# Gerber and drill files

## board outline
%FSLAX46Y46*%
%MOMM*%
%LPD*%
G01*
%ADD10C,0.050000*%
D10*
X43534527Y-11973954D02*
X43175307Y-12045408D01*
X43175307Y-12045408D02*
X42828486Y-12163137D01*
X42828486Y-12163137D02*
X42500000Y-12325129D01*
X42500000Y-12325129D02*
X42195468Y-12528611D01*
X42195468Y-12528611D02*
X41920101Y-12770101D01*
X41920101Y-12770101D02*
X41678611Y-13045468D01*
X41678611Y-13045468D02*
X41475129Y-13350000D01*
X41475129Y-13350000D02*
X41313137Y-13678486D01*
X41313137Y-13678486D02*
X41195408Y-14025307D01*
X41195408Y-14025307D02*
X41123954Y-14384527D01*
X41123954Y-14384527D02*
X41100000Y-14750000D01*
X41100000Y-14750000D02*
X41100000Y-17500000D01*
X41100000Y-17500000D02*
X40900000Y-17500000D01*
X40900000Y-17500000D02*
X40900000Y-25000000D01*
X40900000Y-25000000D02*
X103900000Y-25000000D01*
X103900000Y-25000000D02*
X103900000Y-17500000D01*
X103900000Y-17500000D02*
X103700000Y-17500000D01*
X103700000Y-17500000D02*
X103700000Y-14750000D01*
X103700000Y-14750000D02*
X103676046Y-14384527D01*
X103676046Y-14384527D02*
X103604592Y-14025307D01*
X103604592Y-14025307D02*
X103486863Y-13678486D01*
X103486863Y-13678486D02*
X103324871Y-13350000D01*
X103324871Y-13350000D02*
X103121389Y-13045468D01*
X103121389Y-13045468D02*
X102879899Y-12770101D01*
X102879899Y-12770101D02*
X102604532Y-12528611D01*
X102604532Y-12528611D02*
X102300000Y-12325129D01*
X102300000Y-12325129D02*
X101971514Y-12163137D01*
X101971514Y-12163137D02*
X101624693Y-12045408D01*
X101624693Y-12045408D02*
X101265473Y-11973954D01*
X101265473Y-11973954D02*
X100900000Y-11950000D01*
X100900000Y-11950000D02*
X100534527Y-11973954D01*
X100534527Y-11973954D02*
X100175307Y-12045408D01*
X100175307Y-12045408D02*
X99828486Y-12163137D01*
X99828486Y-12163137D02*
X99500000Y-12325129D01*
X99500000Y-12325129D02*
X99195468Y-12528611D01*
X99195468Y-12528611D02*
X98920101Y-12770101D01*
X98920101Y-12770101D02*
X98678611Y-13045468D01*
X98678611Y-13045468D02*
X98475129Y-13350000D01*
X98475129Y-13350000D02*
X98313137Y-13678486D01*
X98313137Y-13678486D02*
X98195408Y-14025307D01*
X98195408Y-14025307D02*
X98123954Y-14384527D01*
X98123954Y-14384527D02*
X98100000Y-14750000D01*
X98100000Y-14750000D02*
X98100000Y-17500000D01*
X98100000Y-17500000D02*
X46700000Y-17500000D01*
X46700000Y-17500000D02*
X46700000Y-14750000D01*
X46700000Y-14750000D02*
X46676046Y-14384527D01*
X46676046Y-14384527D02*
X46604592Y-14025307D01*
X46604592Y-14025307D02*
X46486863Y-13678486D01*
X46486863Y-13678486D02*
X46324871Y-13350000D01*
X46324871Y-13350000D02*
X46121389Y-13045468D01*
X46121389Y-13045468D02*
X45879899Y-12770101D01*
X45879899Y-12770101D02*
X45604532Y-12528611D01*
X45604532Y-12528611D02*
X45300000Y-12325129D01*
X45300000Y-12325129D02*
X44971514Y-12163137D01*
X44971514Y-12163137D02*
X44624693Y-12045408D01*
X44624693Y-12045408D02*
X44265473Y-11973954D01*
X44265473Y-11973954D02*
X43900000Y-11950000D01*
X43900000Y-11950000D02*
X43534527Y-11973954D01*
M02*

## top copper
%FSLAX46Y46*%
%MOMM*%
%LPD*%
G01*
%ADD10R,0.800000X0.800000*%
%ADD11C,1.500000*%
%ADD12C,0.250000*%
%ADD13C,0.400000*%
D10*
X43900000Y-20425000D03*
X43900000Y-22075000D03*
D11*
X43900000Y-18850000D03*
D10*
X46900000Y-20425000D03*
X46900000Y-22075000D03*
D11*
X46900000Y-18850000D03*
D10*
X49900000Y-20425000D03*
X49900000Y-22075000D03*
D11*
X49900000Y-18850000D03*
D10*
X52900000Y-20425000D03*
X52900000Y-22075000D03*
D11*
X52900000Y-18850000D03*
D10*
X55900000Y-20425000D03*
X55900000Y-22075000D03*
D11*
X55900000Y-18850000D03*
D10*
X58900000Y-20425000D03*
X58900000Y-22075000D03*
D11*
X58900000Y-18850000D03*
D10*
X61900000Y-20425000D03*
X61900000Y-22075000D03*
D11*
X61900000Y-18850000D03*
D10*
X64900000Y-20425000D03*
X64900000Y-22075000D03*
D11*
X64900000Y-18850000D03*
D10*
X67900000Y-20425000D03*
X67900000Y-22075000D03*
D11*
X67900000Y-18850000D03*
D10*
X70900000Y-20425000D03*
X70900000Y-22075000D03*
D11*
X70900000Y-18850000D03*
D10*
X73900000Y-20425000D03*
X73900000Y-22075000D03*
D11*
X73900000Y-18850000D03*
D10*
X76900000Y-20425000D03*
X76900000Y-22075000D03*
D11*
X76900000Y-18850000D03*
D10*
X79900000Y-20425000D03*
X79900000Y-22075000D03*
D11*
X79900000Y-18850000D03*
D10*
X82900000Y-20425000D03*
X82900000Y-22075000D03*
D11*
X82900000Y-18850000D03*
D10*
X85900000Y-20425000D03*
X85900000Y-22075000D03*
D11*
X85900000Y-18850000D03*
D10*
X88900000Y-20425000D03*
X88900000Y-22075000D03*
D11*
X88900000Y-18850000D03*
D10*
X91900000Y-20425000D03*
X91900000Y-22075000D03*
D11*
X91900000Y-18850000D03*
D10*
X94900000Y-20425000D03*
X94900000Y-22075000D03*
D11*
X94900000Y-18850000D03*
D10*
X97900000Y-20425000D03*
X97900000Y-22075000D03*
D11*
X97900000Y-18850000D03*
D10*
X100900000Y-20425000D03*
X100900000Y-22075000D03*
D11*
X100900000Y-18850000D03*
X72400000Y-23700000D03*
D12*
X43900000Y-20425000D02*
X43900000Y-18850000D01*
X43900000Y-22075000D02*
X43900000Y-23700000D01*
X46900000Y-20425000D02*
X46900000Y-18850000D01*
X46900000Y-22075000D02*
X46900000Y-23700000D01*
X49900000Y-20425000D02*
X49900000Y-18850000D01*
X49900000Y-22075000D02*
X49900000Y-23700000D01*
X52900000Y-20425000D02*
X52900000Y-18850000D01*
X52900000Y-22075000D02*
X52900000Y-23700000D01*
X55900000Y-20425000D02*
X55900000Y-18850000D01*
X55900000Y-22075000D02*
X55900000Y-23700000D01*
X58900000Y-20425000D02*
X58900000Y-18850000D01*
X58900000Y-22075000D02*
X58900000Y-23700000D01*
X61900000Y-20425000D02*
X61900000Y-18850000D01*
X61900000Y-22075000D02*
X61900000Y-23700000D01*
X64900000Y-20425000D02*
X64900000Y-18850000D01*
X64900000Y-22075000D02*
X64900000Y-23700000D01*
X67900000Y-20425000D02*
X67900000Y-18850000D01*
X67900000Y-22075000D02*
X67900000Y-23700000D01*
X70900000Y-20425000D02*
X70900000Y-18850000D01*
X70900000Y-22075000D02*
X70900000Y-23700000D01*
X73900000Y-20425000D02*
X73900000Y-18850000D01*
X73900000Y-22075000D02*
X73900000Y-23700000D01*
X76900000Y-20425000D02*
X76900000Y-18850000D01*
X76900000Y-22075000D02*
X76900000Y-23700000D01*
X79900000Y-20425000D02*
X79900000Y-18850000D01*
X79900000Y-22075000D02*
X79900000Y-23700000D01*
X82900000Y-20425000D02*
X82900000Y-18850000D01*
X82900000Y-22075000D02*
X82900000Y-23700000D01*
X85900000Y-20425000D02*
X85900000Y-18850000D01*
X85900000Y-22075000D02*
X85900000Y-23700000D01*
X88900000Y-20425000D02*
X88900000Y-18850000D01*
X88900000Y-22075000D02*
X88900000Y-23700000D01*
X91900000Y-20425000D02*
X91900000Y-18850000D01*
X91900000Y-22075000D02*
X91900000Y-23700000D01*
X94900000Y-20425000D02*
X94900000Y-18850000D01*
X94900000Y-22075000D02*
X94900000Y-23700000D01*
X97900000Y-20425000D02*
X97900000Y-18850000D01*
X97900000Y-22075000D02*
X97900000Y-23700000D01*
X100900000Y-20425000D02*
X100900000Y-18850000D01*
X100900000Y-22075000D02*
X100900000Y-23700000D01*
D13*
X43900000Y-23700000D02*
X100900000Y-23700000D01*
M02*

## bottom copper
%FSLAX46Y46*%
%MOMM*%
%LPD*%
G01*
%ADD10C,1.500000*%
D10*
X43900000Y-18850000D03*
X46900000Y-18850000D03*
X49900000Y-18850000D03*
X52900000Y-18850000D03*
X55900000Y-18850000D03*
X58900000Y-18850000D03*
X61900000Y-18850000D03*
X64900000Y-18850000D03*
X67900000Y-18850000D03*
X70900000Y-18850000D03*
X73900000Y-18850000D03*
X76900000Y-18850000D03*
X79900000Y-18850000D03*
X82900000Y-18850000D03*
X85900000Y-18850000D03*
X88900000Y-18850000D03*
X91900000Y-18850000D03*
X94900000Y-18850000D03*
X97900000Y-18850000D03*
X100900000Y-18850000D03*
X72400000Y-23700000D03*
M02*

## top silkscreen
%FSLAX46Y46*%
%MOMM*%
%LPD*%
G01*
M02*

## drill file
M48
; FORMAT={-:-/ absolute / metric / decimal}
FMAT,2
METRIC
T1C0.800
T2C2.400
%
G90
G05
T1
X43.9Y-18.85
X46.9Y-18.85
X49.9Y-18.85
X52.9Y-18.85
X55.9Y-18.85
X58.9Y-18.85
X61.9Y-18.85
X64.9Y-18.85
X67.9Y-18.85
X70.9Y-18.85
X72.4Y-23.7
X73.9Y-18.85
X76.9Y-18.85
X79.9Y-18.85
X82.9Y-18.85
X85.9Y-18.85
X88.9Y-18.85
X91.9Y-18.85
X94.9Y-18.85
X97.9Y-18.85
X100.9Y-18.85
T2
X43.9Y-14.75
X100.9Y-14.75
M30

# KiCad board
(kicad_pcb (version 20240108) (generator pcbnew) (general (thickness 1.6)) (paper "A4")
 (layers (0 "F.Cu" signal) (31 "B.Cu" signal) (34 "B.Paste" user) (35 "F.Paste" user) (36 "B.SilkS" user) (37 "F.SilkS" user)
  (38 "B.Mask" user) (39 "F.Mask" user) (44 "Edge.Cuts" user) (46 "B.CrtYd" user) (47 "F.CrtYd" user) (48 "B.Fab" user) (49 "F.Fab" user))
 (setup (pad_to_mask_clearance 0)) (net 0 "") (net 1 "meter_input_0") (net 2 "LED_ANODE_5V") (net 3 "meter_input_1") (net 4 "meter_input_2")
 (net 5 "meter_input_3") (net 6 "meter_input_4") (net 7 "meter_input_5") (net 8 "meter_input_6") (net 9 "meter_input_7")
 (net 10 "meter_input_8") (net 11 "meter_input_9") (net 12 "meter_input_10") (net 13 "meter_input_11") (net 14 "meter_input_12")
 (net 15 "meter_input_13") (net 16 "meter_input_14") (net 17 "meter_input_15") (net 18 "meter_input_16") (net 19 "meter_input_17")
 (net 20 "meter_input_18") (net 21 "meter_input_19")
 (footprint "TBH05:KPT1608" (layer "F.Cu") (at 43.9 21.25)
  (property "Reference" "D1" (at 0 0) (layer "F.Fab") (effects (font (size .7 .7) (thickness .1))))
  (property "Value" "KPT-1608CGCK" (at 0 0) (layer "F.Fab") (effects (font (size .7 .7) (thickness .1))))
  (pad "1" smd rect (at 0 -.825) (size .8 .8) (layers "F.Cu" "F.Paste" "F.Mask") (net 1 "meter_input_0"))
  (pad "2" smd rect (at 0 .825) (size .8 .8) (layers "F.Cu" "F.Paste" "F.Mask") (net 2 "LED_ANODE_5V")))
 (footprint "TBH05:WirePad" (layer "F.Cu") (at 43.9 18.85)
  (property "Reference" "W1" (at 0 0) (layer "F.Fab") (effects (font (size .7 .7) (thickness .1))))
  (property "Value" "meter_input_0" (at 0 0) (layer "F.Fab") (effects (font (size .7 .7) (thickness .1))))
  (pad "1" thru_hole circle (at 0 0) (size 1.5 1.5) (drill .8) (layers "*.Cu" "*.Mask") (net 1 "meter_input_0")))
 (segment (start 43.9 20.425) (end 43.9 18.85) (width 0.25) (layer "F.Cu") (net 1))
 (segment (start 43.9 22.075) (end 43.9 23.7) (width 0.25) (layer "F.Cu") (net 2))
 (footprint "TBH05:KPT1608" (layer "F.Cu") (at 46.9 21.25)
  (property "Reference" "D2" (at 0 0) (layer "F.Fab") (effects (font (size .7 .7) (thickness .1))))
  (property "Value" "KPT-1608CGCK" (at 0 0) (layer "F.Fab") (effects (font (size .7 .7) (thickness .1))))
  (pad "1" smd rect (at 0 -.825) (size .8 .8) (layers "F.Cu" "F.Paste" "F.Mask") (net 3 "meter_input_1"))
  (pad "2" smd rect (at 0 .825) (size .8 .8) (layers "F.Cu" "F.Paste" "F.Mask") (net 2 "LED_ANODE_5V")))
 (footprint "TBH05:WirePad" (layer "F.Cu") (at 46.9 18.85)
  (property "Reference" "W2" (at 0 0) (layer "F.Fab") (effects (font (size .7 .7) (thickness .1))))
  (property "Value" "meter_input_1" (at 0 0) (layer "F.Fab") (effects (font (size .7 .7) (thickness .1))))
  (pad "1" thru_hole circle (at 0 0) (size 1.5 1.5) (drill .8) (layers "*.Cu" "*.Mask") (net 3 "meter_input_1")))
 (segment (start 46.9 20.425) (end 46.9 18.85) (width 0.25) (layer "F.Cu") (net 3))
 (segment (start 46.9 22.075) (end 46.9 23.7) (width 0.25) (layer "F.Cu") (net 2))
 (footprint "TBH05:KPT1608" (layer "F.Cu") (at 49.9 21.25)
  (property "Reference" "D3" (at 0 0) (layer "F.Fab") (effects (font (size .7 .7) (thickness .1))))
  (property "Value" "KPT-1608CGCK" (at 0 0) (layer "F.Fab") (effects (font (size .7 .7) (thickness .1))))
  (pad "1" smd rect (at 0 -.825) (size .8 .8) (layers "F.Cu" "F.Paste" "F.Mask") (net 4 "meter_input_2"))
  (pad "2" smd rect (at 0 .825) (size .8 .8) (layers "F.Cu" "F.Paste" "F.Mask") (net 2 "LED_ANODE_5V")))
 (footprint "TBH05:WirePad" (layer "F.Cu") (at 49.9 18.85)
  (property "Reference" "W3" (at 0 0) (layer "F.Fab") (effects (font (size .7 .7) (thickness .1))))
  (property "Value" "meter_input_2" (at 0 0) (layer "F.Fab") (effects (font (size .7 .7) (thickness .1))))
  (pad "1" thru_hole circle (at 0 0) (size 1.5 1.5) (drill .8) (layers "*.Cu" "*.Mask") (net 4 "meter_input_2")))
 (segment (start 49.9 20.425) (end 49.9 18.85) (width 0.25) (layer "F.Cu") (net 4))
 (segment (start 49.9 22.075) (end 49.9 23.7) (width 0.25) (layer "F.Cu") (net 2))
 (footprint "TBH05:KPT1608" (layer "F.Cu") (at 52.9 21.25)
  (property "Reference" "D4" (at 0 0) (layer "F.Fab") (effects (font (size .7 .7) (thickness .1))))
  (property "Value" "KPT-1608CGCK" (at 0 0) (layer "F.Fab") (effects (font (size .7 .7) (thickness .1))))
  (pad "1" smd rect (at 0 -.825) (size .8 .8) (layers "F.Cu" "F.Paste" "F.Mask") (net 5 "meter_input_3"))
  (pad "2" smd rect (at 0 .825) (size .8 .8) (layers "F.Cu" "F.Paste" "F.Mask") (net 2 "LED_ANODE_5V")))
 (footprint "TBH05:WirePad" (layer "F.Cu") (at 52.9 18.85)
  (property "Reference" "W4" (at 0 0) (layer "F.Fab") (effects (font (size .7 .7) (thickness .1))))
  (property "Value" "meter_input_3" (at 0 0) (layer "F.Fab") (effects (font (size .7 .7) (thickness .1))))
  (pad "1" thru_hole circle (at 0 0) (size 1.5 1.5) (drill .8) (layers "*.Cu" "*.Mask") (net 5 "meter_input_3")))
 (segment (start 52.9 20.425) (end 52.9 18.85) (width 0.25) (layer "F.Cu") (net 5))
 (segment (start 52.9 22.075) (end 52.9 23.7) (width 0.25) (layer "F.Cu") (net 2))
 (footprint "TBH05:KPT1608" (layer "F.Cu") (at 55.9 21.25)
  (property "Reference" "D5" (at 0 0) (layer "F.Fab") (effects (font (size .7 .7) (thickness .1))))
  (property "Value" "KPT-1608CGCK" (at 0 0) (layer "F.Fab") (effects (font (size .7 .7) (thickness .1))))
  (pad "1" smd rect (at 0 -.825) (size .8 .8) (layers "F.Cu" "F.Paste" "F.Mask") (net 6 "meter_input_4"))
  (pad "2" smd rect (at 0 .825) (size .8 .8) (layers "F.Cu" "F.Paste" "F.Mask") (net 2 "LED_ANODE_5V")))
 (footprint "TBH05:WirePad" (layer "F.Cu") (at 55.9 18.85)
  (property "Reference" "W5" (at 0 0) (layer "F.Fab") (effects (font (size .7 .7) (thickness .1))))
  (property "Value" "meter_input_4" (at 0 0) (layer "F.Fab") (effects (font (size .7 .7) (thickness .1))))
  (pad "1" thru_hole circle (at 0 0) (size 1.5 1.5) (drill .8) (layers "*.Cu" "*.Mask") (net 6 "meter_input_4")))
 (segment (start 55.9 20.425) (end 55.9 18.85) (width 0.25) (layer "F.Cu") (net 6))
 (segment (start 55.9 22.075) (end 55.9 23.7) (width 0.25) (layer "F.Cu") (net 2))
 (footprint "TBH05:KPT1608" (layer "F.Cu") (at 58.9 21.25)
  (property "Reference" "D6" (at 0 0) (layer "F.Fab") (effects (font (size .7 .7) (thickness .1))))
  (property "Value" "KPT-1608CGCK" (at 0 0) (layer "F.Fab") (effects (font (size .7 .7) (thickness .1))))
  (pad "1" smd rect (at 0 -.825) (size .8 .8) (layers "F.Cu" "F.Paste" "F.Mask") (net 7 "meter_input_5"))
  (pad "2" smd rect (at 0 .825) (size .8 .8) (layers "F.Cu" "F.Paste" "F.Mask") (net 2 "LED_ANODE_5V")))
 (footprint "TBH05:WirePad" (layer "F.Cu") (at 58.9 18.85)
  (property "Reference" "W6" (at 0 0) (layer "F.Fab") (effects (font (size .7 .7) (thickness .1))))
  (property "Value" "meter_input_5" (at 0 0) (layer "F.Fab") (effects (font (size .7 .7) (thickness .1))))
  (pad "1" thru_hole circle (at 0 0) (size 1.5 1.5) (drill .8) (layers "*.Cu" "*.Mask") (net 7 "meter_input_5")))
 (segment (start 58.9 20.425) (end 58.9 18.85) (width 0.25) (layer "F.Cu") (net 7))
 (segment (start 58.9 22.075) (end 58.9 23.7) (width 0.25) (layer "F.Cu") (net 2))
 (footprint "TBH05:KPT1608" (layer "F.Cu") (at 61.9 21.25)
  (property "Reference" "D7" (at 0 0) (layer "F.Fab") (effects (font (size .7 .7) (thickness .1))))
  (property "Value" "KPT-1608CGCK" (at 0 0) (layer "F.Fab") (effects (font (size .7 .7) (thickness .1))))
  (pad "1" smd rect (at 0 -.825) (size .8 .8) (layers "F.Cu" "F.Paste" "F.Mask") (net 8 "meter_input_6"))
  (pad "2" smd rect (at 0 .825) (size .8 .8) (layers "F.Cu" "F.Paste" "F.Mask") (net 2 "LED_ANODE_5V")))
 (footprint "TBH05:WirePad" (layer "F.Cu") (at 61.9 18.85)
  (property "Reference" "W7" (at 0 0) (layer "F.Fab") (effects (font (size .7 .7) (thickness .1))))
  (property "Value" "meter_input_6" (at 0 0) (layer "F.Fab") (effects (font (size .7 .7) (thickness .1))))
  (pad "1" thru_hole circle (at 0 0) (size 1.5 1.5) (drill .8) (layers "*.Cu" "*.Mask") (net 8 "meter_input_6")))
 (segment (start 61.9 20.425) (end 61.9 18.85) (width 0.25) (layer "F.Cu") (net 8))
 (segment (start 61.9 22.075) (end 61.9 23.7) (width 0.25) (layer "F.Cu") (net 2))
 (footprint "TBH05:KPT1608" (layer "F.Cu") (at 64.9 21.25)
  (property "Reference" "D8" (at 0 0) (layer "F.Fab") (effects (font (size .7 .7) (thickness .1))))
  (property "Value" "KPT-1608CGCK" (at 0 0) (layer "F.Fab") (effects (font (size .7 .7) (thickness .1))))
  (pad "1" smd rect (at 0 -.825) (size .8 .8) (layers "F.Cu" "F.Paste" "F.Mask") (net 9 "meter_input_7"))
  (pad "2" smd rect (at 0 .825) (size .8 .8) (layers "F.Cu" "F.Paste" "F.Mask") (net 2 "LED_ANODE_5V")))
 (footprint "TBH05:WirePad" (layer "F.Cu") (at 64.9 18.85)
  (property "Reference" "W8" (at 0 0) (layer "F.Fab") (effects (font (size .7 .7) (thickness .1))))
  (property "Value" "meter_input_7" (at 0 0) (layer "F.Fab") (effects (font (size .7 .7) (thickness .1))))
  (pad "1" thru_hole circle (at 0 0) (size 1.5 1.5) (drill .8) (layers "*.Cu" "*.Mask") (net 9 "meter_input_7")))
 (segment (start 64.9 20.425) (end 64.9 18.85) (width 0.25) (layer "F.Cu") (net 9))
 (segment (start 64.9 22.075) (end 64.9 23.7) (width 0.25) (layer "F.Cu") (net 2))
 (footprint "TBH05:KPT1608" (layer "F.Cu") (at 67.9 21.25)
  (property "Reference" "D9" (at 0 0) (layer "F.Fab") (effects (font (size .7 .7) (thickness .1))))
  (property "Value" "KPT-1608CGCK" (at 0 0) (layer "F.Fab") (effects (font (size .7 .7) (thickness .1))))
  (pad "1" smd rect (at 0 -.825) (size .8 .8) (layers "F.Cu" "F.Paste" "F.Mask") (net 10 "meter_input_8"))
  (pad "2" smd rect (at 0 .825) (size .8 .8) (layers "F.Cu" "F.Paste" "F.Mask") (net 2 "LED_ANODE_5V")))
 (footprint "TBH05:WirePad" (layer "F.Cu") (at 67.9 18.85)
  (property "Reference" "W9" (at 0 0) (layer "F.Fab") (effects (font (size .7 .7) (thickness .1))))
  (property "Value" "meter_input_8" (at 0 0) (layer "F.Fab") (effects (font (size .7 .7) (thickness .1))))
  (pad "1" thru_hole circle (at 0 0) (size 1.5 1.5) (drill .8) (layers "*.Cu" "*.Mask") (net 10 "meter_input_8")))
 (segment (start 67.9 20.425) (end 67.9 18.85) (width 0.25) (layer "F.Cu") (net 10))
 (segment (start 67.9 22.075) (end 67.9 23.7) (width 0.25) (layer "F.Cu") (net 2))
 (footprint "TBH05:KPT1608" (layer "F.Cu") (at 70.9 21.25)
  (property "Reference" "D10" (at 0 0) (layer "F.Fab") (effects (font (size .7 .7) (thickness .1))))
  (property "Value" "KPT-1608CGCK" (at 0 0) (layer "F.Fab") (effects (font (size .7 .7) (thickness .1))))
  (pad "1" smd rect (at 0 -.825) (size .8 .8) (layers "F.Cu" "F.Paste" "F.Mask") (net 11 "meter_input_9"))
  (pad "2" smd rect (at 0 .825) (size .8 .8) (layers "F.Cu" "F.Paste" "F.Mask") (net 2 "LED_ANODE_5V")))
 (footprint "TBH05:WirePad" (layer "F.Cu") (at 70.9 18.85)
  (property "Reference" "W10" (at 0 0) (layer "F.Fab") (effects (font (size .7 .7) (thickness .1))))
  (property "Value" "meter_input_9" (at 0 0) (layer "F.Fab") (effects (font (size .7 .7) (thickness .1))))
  (pad "1" thru_hole circle (at 0 0) (size 1.5 1.5) (drill .8) (layers "*.Cu" "*.Mask") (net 11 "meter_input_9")))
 (segment (start 70.9 20.425) (end 70.9 18.85) (width 0.25) (layer "F.Cu") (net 11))
 (segment (start 70.9 22.075) (end 70.9 23.7) (width 0.25) (layer "F.Cu") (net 2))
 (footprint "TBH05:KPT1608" (layer "F.Cu") (at 73.9 21.25)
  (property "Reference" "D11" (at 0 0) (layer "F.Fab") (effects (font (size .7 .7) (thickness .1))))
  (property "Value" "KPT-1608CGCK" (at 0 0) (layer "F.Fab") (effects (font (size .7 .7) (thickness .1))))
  (pad "1" smd rect (at 0 -.825) (size .8 .8) (layers "F.Cu" "F.Paste" "F.Mask") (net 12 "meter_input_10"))
  (pad "2" smd rect (at 0 .825) (size .8 .8) (layers "F.Cu" "F.Paste" "F.Mask") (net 2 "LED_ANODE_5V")))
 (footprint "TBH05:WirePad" (layer "F.Cu") (at 73.9 18.85)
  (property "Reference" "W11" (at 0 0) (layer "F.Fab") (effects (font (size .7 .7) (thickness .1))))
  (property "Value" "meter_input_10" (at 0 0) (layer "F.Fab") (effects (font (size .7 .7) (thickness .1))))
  (pad "1" thru_hole circle (at 0 0) (size 1.5 1.5) (drill .8) (layers "*.Cu" "*.Mask") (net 12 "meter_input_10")))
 (segment (start 73.9 20.425) (end 73.9 18.85) (width 0.25) (layer "F.Cu") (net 12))
 (segment (start 73.9 22.075) (end 73.9 23.7) (width 0.25) (layer "F.Cu") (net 2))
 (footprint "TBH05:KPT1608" (layer "F.Cu") (at 76.9 21.25)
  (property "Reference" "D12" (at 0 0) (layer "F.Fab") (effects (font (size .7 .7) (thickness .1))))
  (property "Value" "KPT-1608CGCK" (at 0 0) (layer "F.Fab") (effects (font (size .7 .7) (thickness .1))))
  (pad "1" smd rect (at 0 -.825) (size .8 .8) (layers "F.Cu" "F.Paste" "F.Mask") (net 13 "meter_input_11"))
  (pad "2" smd rect (at 0 .825) (size .8 .8) (layers "F.Cu" "F.Paste" "F.Mask") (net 2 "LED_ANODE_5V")))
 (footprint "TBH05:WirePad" (layer "F.Cu") (at 76.9 18.85)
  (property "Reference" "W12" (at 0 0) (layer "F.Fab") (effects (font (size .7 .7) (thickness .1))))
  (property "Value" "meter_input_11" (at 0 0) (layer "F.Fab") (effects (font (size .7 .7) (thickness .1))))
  (pad "1" thru_hole circle (at 0 0) (size 1.5 1.5) (drill .8) (layers "*.Cu" "*.Mask") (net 13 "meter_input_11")))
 (segment (start 76.9 20.425) (end 76.9 18.85) (width 0.25) (layer "F.Cu") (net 13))
 (segment (start 76.9 22.075) (end 76.9 23.7) (width 0.25) (layer "F.Cu") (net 2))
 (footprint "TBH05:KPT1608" (layer "F.Cu") (at 79.9 21.25)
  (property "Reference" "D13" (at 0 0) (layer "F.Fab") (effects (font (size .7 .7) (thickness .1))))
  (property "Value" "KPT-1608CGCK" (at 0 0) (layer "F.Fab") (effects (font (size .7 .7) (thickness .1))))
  (pad "1" smd rect (at 0 -.825) (size .8 .8) (layers "F.Cu" "F.Paste" "F.Mask") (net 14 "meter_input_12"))
  (pad "2" smd rect (at 0 .825) (size .8 .8) (layers "F.Cu" "F.Paste" "F.Mask") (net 2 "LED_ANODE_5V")))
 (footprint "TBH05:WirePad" (layer "F.Cu") (at 79.9 18.85)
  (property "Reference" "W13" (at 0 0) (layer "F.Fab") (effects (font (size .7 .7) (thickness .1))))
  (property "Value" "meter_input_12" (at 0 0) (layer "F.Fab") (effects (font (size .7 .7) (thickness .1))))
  (pad "1" thru_hole circle (at 0 0) (size 1.5 1.5) (drill .8) (layers "*.Cu" "*.Mask") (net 14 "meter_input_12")))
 (segment (start 79.9 20.425) (end 79.9 18.85) (width 0.25) (layer "F.Cu") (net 14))
 (segment (start 79.9 22.075) (end 79.9 23.7) (width 0.25) (layer "F.Cu") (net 2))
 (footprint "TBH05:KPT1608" (layer "F.Cu") (at 82.9 21.25)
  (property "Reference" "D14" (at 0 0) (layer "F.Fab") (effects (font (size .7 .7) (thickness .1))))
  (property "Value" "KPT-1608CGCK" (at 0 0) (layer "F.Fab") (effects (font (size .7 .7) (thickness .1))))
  (pad "1" smd rect (at 0 -.825) (size .8 .8) (layers "F.Cu" "F.Paste" "F.Mask") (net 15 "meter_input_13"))
  (pad "2" smd rect (at 0 .825) (size .8 .8) (layers "F.Cu" "F.Paste" "F.Mask") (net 2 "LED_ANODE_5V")))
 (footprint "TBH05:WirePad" (layer "F.Cu") (at 82.9 18.85)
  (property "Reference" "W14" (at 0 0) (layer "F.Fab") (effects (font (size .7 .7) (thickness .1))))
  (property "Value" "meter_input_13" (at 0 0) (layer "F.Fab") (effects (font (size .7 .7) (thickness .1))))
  (pad "1" thru_hole circle (at 0 0) (size 1.5 1.5) (drill .8) (layers "*.Cu" "*.Mask") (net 15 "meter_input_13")))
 (segment (start 82.9 20.425) (end 82.9 18.85) (width 0.25) (layer "F.Cu") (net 15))
 (segment (start 82.9 22.075) (end 82.9 23.7) (width 0.25) (layer "F.Cu") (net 2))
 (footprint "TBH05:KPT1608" (layer "F.Cu") (at 85.9 21.25)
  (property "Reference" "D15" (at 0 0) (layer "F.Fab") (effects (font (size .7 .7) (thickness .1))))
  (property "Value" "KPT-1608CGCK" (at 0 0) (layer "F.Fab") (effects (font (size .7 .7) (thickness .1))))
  (pad "1" smd rect (at 0 -.825) (size .8 .8) (layers "F.Cu" "F.Paste" "F.Mask") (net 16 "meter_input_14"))
  (pad "2" smd rect (at 0 .825) (size .8 .8) (layers "F.Cu" "F.Paste" "F.Mask") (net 2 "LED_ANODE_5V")))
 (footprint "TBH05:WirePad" (layer "F.Cu") (at 85.9 18.85)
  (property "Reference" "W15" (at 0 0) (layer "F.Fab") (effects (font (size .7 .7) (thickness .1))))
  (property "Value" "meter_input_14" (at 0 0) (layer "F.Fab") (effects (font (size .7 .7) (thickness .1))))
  (pad "1" thru_hole circle (at 0 0) (size 1.5 1.5) (drill .8) (layers "*.Cu" "*.Mask") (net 16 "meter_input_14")))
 (segment (start 85.9 20.425) (end 85.9 18.85) (width 0.25) (layer "F.Cu") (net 16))
 (segment (start 85.9 22.075) (end 85.9 23.7) (width 0.25) (layer "F.Cu") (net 2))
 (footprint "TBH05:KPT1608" (layer "F.Cu") (at 88.9 21.25)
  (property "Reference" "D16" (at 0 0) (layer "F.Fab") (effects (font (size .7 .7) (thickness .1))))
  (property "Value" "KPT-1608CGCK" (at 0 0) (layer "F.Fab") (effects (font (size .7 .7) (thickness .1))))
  (pad "1" smd rect (at 0 -.825) (size .8 .8) (layers "F.Cu" "F.Paste" "F.Mask") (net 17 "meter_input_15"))
  (pad "2" smd rect (at 0 .825) (size .8 .8) (layers "F.Cu" "F.Paste" "F.Mask") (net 2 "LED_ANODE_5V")))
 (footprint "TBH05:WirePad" (layer "F.Cu") (at 88.9 18.85)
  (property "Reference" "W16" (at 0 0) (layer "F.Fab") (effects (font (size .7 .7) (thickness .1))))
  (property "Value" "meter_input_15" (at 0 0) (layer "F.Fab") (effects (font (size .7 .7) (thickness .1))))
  (pad "1" thru_hole circle (at 0 0) (size 1.5 1.5) (drill .8) (layers "*.Cu" "*.Mask") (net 17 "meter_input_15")))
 (segment (start 88.9 20.425) (end 88.9 18.85) (width 0.25) (layer "F.Cu") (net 17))
 (segment (start 88.9 22.075) (end 88.9 23.7) (width 0.25) (layer "F.Cu") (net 2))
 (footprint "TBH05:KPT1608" (layer "F.Cu") (at 91.9 21.25)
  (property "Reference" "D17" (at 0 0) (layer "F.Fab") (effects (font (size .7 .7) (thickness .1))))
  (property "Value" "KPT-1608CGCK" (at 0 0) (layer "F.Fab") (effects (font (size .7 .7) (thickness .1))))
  (pad "1" smd rect (at 0 -.825) (size .8 .8) (layers "F.Cu" "F.Paste" "F.Mask") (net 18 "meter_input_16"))
  (pad "2" smd rect (at 0 .825) (size .8 .8) (layers "F.Cu" "F.Paste" "F.Mask") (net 2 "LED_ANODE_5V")))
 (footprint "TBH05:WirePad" (layer "F.Cu") (at 91.9 18.85)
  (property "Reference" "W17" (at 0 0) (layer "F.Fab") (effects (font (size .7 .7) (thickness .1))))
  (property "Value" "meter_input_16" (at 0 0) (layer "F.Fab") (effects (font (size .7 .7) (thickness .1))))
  (pad "1" thru_hole circle (at 0 0) (size 1.5 1.5) (drill .8) (layers "*.Cu" "*.Mask") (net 18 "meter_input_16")))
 (segment (start 91.9 20.425) (end 91.9 18.85) (width 0.25) (layer "F.Cu") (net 18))
 (segment (start 91.9 22.075) (end 91.9 23.7) (width 0.25) (layer "F.Cu") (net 2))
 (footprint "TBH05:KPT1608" (layer "F.Cu") (at 94.9 21.25)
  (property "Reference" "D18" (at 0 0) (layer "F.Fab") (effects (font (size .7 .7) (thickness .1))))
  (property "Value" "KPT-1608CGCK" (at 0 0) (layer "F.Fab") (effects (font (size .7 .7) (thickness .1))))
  (pad "1" smd rect (at 0 -.825) (size .8 .8) (layers "F.Cu" "F.Paste" "F.Mask") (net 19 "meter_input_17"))
  (pad "2" smd rect (at 0 .825) (size .8 .8) (layers "F.Cu" "F.Paste" "F.Mask") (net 2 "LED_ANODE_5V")))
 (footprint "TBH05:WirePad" (layer "F.Cu") (at 94.9 18.85)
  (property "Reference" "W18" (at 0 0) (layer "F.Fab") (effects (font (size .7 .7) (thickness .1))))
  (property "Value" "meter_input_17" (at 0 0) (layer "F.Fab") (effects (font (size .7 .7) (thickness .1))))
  (pad "1" thru_hole circle (at 0 0) (size 1.5 1.5) (drill .8) (layers "*.Cu" "*.Mask") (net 19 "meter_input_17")))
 (segment (start 94.9 20.425) (end 94.9 18.85) (width 0.25) (layer "F.Cu") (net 19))
 (segment (start 94.9 22.075) (end 94.9 23.7) (width 0.25) (layer "F.Cu") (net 2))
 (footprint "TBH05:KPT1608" (layer "F.Cu") (at 97.9 21.25)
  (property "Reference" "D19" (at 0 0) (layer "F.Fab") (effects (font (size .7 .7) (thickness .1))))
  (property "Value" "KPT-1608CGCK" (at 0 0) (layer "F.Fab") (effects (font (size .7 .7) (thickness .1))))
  (pad "1" smd rect (at 0 -.825) (size .8 .8) (layers "F.Cu" "F.Paste" "F.Mask") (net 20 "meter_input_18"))
  (pad "2" smd rect (at 0 .825) (size .8 .8) (layers "F.Cu" "F.Paste" "F.Mask") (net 2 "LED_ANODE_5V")))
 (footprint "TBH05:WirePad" (layer "F.Cu") (at 97.9 18.85)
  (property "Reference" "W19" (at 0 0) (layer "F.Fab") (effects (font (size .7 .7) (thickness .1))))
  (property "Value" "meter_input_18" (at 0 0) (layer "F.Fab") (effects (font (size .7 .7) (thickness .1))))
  (pad "1" thru_hole circle (at 0 0) (size 1.5 1.5) (drill .8) (layers "*.Cu" "*.Mask") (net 20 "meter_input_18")))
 (segment (start 97.9 20.425) (end 97.9 18.85) (width 0.25) (layer "F.Cu") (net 20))
 (segment (start 97.9 22.075) (end 97.9 23.7) (width 0.25) (layer "F.Cu") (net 2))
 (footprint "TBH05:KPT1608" (layer "F.Cu") (at 100.9 21.25)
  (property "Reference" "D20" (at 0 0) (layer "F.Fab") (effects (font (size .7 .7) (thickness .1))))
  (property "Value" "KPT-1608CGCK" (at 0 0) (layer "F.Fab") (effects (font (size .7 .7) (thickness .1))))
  (pad "1" smd rect (at 0 -.825) (size .8 .8) (layers "F.Cu" "F.Paste" "F.Mask") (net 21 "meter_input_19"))
  (pad "2" smd rect (at 0 .825) (size .8 .8) (layers "F.Cu" "F.Paste" "F.Mask") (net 2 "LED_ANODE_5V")))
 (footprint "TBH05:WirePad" (layer "F.Cu") (at 100.9 18.85)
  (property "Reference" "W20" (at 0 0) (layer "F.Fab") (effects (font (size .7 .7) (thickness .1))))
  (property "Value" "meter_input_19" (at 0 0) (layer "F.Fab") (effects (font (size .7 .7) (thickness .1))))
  (pad "1" thru_hole circle (at 0 0) (size 1.5 1.5) (drill .8) (layers "*.Cu" "*.Mask") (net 21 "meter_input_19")))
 (segment (start 100.9 20.425) (end 100.9 18.85) (width 0.25) (layer "F.Cu") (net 21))
 (segment (start 100.9 22.075) (end 100.9 23.7) (width 0.25) (layer "F.Cu") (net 2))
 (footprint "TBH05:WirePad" (layer "F.Cu") (at 72.4 23.7)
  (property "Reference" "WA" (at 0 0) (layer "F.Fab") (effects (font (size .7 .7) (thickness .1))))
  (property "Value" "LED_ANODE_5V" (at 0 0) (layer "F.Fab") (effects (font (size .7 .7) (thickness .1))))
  (pad "1" thru_hole circle (at 0 0) (size 1.5 1.5) (drill .8) (layers "*.Cu" "*.Mask") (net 2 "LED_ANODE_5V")))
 (segment (start 43.9 23.7) (end 100.9 23.7) (width 0.4) (layer "F.Cu") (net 2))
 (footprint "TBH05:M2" (layer "F.Cu") (at 43.9 14.75)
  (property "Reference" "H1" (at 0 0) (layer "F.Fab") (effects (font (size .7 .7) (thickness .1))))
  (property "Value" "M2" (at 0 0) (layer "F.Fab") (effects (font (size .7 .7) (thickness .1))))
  (pad "" np_thru_hole circle (at 0 0) (size 2.4 2.4) (drill 2.4) (layers "*.Cu" "*.Mask")))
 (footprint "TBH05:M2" (layer "F.Cu") (at 100.9 14.75)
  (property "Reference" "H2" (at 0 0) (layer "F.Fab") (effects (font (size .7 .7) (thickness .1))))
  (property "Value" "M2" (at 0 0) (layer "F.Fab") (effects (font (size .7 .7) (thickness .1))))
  (pad "" np_thru_hole circle (at 0 0) (size 2.4 2.4) (drill 2.4) (layers "*.Cu" "*.Mask")))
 (gr_line (start 43.534527 11.973954) (end 43.175307 12.045408) (stroke (width .05) (type default)) (layer "Edge.Cuts"))
 (gr_line (start 43.175307 12.045408) (end 42.828486 12.163137) (stroke (width .05) (type default)) (layer "Edge.Cuts"))
 (gr_line (start 42.828486 12.163137) (end 42.5 12.325129) (stroke (width .05) (type default)) (layer "Edge.Cuts"))
 (gr_line (start 42.5 12.325129) (end 42.195468 12.528611) (stroke (width .05) (type default)) (layer "Edge.Cuts"))
 (gr_line (start 42.195468 12.528611) (end 41.920101 12.770101) (stroke (width .05) (type default)) (layer "Edge.Cuts"))
 (gr_line (start 41.920101 12.770101) (end 41.678611 13.045468) (stroke (width .05) (type default)) (layer "Edge.Cuts"))
 (gr_line (start 41.678611 13.045468) (end 41.475129 13.35) (stroke (width .05) (type default)) (layer "Edge.Cuts"))
 (gr_line (start 41.475129 13.35) (end 41.313137 13.678486) (stroke (width .05) (type default)) (layer "Edge.Cuts"))
 (gr_line (start 41.313137 13.678486) (end 41.195408 14.025307) (stroke (width .05) (type default)) (layer "Edge.Cuts"))
 (gr_line (start 41.195408 14.025307) (end 41.123954 14.384527) (stroke (width .05) (type default)) (layer "Edge.Cuts"))
 (gr_line (start 41.123954 14.384527) (end 41.1 14.75) (stroke (width .05) (type default)) (layer "Edge.Cuts"))
 (gr_line (start 41.1 14.75) (end 41.1 17.5) (stroke (width .05) (type default)) (layer "Edge.Cuts"))
 (gr_line (start 41.1 17.5) (end 40.9 17.5) (stroke (width .05) (type default)) (layer "Edge.Cuts"))
 (gr_line (start 40.9 17.5) (end 40.9 25.0) (stroke (width .05) (type default)) (layer "Edge.Cuts"))
 (gr_line (start 40.9 25.0) (end 103.9 25.0) (stroke (width .05) (type default)) (layer "Edge.Cuts"))
 (gr_line (start 103.9 25.0) (end 103.9 17.5) (stroke (width .05) (type default)) (layer "Edge.Cuts"))
 (gr_line (start 103.9 17.5) (end 103.7 17.5) (stroke (width .05) (type default)) (layer "Edge.Cuts"))
 (gr_line (start 103.7 17.5) (end 103.7 14.75) (stroke (width .05) (type default)) (layer "Edge.Cuts"))
 (gr_line (start 103.7 14.75) (end 103.676046 14.384527) (stroke (width .05) (type default)) (layer "Edge.Cuts"))
 (gr_line (start 103.676046 14.384527) (end 103.604592 14.025307) (stroke (width .05) (type default)) (layer "Edge.Cuts"))
 (gr_line (start 103.604592 14.025307) (end 103.486863 13.678486) (stroke (width .05) (type default)) (layer "Edge.Cuts"))
 (gr_line (start 103.486863 13.678486) (end 103.324871 13.35) (stroke (width .05) (type default)) (layer "Edge.Cuts"))
 (gr_line (start 103.324871 13.35) (end 103.121389 13.045468) (stroke (width .05) (type default)) (layer "Edge.Cuts"))
 (gr_line (start 103.121389 13.045468) (end 102.879899 12.770101) (stroke (width .05) (type default)) (layer "Edge.Cuts"))
 (gr_line (start 102.879899 12.770101) (end 102.604532 12.528611) (stroke (width .05) (type default)) (layer "Edge.Cuts"))
 (gr_line (start 102.604532 12.528611) (end 102.3 12.325129) (stroke (width .05) (type default)) (layer "Edge.Cuts"))
 (gr_line (start 102.3 12.325129) (end 101.971514 12.163137) (stroke (width .05) (type default)) (layer "Edge.Cuts"))
 (gr_line (start 101.971514 12.163137) (end 101.624693 12.045408) (stroke (width .05) (type default)) (layer "Edge.Cuts"))
 (gr_line (start 101.624693 12.045408) (end 101.265473 11.973954) (stroke (width .05) (type default)) (layer "Edge.Cuts"))
 (gr_line (start 101.265473 11.973954) (end 100.9 11.95) (stroke (width .05) (type default)) (layer "Edge.Cuts"))
 (gr_line (start 100.9 11.95) (end 100.534527 11.973954) (stroke (width .05) (type default)) (layer "Edge.Cuts"))
 (gr_line (start 100.534527 11.973954) (end 100.175307 12.045408) (stroke (width .05) (type default)) (layer "Edge.Cuts"))
 (gr_line (start 100.175307 12.045408) (end 99.828486 12.163137) (stroke (width .05) (type default)) (layer "Edge.Cuts"))
 (gr_line (start 99.828486 12.163137) (end 99.5 12.325129) (stroke (width .05) (type default)) (layer "Edge.Cuts"))
 (gr_line (start 99.5 12.325129) (end 99.195468 12.528611) (stroke (width .05) (type default)) (layer "Edge.Cuts"))
 (gr_line (start 99.195468 12.528611) (end 98.920101 12.770101) (stroke (width .05) (type default)) (layer "Edge.Cuts"))
 (gr_line (start 98.920101 12.770101) (end 98.678611 13.045468) (stroke (width .05) (type default)) (layer "Edge.Cuts"))
 (gr_line (start 98.678611 13.045468) (end 98.475129 13.35) (stroke (width .05) (type default)) (layer "Edge.Cuts"))
 (gr_line (start 98.475129 13.35) (end 98.313137 13.678486) (stroke (width .05) (type default)) (layer "Edge.Cuts"))
 (gr_line (start 98.313137 13.678486) (end 98.195408 14.025307) (stroke (width .05) (type default)) (layer "Edge.Cuts"))
 (gr_line (start 98.195408 14.025307) (end 98.123954 14.384527) (stroke (width .05) (type default)) (layer "Edge.Cuts"))
 (gr_line (start 98.123954 14.384527) (end 98.1 14.75) (stroke (width .05) (type default)) (layer "Edge.Cuts"))
 (gr_line (start 98.1 14.75) (end 98.1 17.5) (stroke (width .05) (type default)) (layer "Edge.Cuts"))
 (gr_line (start 98.1 17.5) (end 46.7 17.5) (stroke (width .05) (type default)) (layer "Edge.Cuts"))
 (gr_line (start 46.7 17.5) (end 46.7 14.75) (stroke (width .05) (type default)) (layer "Edge.Cuts"))
 (gr_line (start 46.7 14.75) (end 46.676046 14.384527) (stroke (width .05) (type default)) (layer "Edge.Cuts"))
 (gr_line (start 46.676046 14.384527) (end 46.604592 14.025307) (stroke (width .05) (type default)) (layer "Edge.Cuts"))
 (gr_line (start 46.604592 14.025307) (end 46.486863 13.678486) (stroke (width .05) (type default)) (layer "Edge.Cuts"))
 (gr_line (start 46.486863 13.678486) (end 46.324871 13.35) (stroke (width .05) (type default)) (layer "Edge.Cuts"))
 (gr_line (start 46.324871 13.35) (end 46.121389 13.045468) (stroke (width .05) (type default)) (layer "Edge.Cuts"))
 (gr_line (start 46.121389 13.045468) (end 45.879899 12.770101) (stroke (width .05) (type default)) (layer "Edge.Cuts"))
 (gr_line (start 45.879899 12.770101) (end 45.604532 12.528611) (stroke (width .05) (type default)) (layer "Edge.Cuts"))
 (gr_line (start 45.604532 12.528611) (end 45.3 12.325129) (stroke (width .05) (type default)) (layer "Edge.Cuts"))
 (gr_line (start 45.3 12.325129) (end 44.971514 12.163137) (stroke (width .05) (type default)) (layer "Edge.Cuts"))
 (gr_line (start 44.971514 12.163137) (end 44.624693 12.045408) (stroke (width .05) (type default)) (layer "Edge.Cuts"))
 (gr_line (start 44.624693 12.045408) (end 44.265473 11.973954) (stroke (width .05) (type default)) (layer "Edge.Cuts"))
 (gr_line (start 44.265473 11.973954) (end 43.9 11.95) (stroke (width .05) (type default)) (layer "Edge.Cuts"))
 (gr_line (start 43.9 11.95) (end 43.534527 11.973954) (stroke (width .05) (type default)) (layer "Edge.Cuts")))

